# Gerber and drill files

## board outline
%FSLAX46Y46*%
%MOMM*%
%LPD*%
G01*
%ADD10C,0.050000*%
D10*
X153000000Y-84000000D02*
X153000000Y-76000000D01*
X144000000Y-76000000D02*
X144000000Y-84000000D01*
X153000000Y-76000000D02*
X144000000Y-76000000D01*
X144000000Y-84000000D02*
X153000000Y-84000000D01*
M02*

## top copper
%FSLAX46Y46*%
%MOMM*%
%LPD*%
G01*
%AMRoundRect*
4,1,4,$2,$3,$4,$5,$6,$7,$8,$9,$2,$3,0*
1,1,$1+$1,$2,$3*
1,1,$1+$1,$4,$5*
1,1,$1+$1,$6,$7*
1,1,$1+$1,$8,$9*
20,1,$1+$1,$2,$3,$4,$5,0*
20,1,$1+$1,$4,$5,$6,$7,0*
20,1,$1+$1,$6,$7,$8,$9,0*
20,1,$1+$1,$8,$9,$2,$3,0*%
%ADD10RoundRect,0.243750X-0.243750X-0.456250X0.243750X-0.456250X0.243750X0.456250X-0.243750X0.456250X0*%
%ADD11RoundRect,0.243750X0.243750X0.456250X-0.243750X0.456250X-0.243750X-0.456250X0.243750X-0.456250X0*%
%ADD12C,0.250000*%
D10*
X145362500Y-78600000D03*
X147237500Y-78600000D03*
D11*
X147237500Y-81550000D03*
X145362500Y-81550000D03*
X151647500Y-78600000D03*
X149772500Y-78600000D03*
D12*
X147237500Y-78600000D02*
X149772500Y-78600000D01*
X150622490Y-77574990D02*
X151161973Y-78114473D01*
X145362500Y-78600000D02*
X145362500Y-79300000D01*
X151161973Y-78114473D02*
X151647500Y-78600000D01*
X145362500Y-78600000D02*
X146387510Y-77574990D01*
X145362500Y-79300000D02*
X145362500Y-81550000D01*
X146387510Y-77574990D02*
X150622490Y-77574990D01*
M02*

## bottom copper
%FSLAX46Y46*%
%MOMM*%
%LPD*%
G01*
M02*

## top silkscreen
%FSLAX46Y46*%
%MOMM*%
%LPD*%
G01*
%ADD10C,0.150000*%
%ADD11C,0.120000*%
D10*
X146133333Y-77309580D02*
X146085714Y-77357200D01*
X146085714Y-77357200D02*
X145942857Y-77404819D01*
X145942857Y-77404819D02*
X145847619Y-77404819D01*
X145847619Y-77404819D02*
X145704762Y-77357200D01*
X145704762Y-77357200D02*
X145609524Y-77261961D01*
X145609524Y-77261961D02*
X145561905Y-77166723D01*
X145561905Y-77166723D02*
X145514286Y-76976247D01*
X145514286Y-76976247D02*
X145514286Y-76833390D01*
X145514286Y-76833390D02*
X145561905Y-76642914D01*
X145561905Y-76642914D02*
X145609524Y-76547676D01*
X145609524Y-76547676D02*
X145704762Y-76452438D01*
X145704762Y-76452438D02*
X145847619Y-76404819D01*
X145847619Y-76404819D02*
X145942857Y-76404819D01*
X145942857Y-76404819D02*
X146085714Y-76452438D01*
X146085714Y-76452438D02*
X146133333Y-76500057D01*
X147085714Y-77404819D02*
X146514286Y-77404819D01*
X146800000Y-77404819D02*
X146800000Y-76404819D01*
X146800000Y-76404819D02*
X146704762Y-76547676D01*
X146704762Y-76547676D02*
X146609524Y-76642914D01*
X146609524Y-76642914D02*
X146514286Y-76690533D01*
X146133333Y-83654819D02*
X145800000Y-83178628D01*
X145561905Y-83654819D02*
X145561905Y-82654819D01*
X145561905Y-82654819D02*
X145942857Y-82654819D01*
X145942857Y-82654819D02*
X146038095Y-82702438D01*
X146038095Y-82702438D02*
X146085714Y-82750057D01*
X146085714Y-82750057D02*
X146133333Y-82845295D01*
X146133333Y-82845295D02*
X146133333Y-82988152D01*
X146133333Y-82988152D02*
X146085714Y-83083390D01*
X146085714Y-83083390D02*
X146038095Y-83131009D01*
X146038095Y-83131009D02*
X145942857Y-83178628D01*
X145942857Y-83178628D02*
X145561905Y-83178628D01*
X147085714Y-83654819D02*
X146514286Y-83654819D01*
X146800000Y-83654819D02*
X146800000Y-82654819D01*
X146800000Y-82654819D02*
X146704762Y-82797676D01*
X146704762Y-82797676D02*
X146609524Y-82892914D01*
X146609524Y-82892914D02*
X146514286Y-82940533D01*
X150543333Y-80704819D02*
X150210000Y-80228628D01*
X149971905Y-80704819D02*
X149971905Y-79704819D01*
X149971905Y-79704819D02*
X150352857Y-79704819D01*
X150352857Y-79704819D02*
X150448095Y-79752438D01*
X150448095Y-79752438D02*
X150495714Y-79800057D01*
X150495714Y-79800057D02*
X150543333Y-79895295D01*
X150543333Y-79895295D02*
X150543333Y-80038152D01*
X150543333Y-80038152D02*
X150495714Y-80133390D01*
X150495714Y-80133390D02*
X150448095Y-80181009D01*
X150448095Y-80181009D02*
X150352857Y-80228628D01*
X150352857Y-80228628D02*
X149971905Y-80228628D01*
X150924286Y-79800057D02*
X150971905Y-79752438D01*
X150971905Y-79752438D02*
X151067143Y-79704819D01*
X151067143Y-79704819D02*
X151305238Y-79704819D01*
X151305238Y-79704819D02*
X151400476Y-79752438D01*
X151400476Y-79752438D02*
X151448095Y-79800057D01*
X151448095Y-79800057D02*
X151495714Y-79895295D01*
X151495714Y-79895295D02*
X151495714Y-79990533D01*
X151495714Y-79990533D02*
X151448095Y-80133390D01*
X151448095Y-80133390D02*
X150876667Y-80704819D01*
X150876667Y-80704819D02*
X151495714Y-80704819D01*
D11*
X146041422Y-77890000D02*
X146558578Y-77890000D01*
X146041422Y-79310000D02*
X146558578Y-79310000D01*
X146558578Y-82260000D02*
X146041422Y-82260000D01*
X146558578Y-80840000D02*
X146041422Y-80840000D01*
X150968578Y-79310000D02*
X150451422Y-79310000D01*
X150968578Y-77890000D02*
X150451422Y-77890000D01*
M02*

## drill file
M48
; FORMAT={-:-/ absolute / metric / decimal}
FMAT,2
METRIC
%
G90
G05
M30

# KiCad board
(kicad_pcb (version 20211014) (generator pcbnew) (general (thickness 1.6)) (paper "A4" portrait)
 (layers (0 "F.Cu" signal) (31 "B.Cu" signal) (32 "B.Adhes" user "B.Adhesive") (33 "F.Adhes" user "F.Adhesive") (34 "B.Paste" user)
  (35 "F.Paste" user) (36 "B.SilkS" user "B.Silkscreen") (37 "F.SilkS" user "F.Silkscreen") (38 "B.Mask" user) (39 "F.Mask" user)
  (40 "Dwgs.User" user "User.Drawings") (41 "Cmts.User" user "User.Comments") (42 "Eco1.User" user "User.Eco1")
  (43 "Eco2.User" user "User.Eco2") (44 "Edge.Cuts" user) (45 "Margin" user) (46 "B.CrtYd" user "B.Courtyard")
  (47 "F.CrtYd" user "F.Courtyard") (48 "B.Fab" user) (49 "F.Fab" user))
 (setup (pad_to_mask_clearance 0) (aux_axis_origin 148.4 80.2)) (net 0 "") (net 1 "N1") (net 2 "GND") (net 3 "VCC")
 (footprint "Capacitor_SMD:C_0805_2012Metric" (layer "F.Cu") (at 146.3 78.6)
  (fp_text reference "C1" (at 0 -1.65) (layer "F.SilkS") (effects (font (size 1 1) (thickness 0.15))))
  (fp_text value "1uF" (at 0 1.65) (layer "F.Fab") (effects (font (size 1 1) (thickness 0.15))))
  (fp_line (start -0.258578 -0.71) (end 0.258578 -0.71) (layer "F.SilkS") (width 0.12))
  (fp_line (start -0.258578 0.71) (end 0.258578 0.71) (layer "F.SilkS") (width 0.12))
  (pad "1" smd roundrect locked (at -0.9375 0) (size 0.975 1.4) (layers "F.Cu" "F.Paste" "F.Mask") (roundrect_rratio 0.25) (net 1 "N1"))
  (pad "2" smd roundrect locked (at 0.9375 0) (size 0.975 1.4) (layers "F.Cu" "F.Paste" "F.Mask") (roundrect_rratio 0.25) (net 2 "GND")))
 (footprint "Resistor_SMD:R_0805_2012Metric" (layer "F.Cu") (at 146.3 81.55 180)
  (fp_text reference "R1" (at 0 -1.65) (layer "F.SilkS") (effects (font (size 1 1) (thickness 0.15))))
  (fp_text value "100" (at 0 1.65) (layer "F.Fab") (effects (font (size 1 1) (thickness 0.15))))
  (fp_line (start -0.258578 -0.71) (end 0.258578 -0.71) (layer "F.SilkS") (width 0.12))
  (fp_line (start -0.258578 0.71) (end 0.258578 0.71) (layer "F.SilkS") (width 0.12))
  (pad "1" smd roundrect locked (at -0.9375 0 180) (size 0.975 1.4) (layers "F.Cu" "F.Paste" "F.Mask") (roundrect_rratio 0.25) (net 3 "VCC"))
  (pad "2" smd roundrect locked (at 0.9375 0 180) (size 0.975 1.4) (layers "F.Cu" "F.Paste" "F.Mask") (roundrect_rratio 0.25) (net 1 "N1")))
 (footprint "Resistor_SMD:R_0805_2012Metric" (layer "F.Cu") (at 150.71 78.6 180)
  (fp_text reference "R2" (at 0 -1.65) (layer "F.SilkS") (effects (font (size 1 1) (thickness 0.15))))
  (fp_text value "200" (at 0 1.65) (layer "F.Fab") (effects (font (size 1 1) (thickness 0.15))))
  (fp_line (start -0.258578 -0.71) (end 0.258578 -0.71) (layer "F.SilkS") (width 0.12))
  (fp_line (start -0.258578 0.71) (end 0.258578 0.71) (layer "F.SilkS") (width 0.12))
  (pad "1" smd roundrect locked (at -0.9375 0 180) (size 0.975 1.4) (layers "F.Cu" "F.Paste" "F.Mask") (roundrect_rratio 0.25) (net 1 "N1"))
  (pad "2" smd roundrect locked (at 0.9375 0 180) (size 0.975 1.4) (layers "F.Cu" "F.Paste" "F.Mask") (roundrect_rratio 0.25) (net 2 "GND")))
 (gr_line (start 153 84) (end 153 76) (layer "Edge.Cuts") (width 0.05))
 (gr_line (start 144 76) (end 144 84) (layer "Edge.Cuts") (width 0.05))
 (gr_line (start 153 76) (end 144 76) (layer "Edge.Cuts") (width 0.05))
 (gr_line (start 144 84) (end 153 84) (layer "Edge.Cuts") (width 0.05))
 (segment (start 147.2375 78.6) (end 149.7725 78.6) (width 0.25) (layer "F.Cu") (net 2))
 (segment (start 150.62249 77.57499) (end 151.161973 78.114473) (width 0.25) (layer "F.Cu") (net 1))
 (segment (start 145.3625 78.6) (end 145.3625 79.3) (width 0.25) (layer "F.Cu") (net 1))
 (segment (start 151.161973 78.114473) (end 151.6475 78.6) (width 0.25) (layer "F.Cu") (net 1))
 (segment (start 145.3625 78.6) (end 146.38751 77.57499) (width 0.25) (layer "F.Cu") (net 1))
 (segment (start 145.3625 79.3) (end 145.3625 81.55) (width 0.25) (layer "F.Cu") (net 1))
 (segment (start 146.38751 77.57499) (end 150.62249 77.57499) (width 0.25) (layer "F.Cu") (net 1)))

